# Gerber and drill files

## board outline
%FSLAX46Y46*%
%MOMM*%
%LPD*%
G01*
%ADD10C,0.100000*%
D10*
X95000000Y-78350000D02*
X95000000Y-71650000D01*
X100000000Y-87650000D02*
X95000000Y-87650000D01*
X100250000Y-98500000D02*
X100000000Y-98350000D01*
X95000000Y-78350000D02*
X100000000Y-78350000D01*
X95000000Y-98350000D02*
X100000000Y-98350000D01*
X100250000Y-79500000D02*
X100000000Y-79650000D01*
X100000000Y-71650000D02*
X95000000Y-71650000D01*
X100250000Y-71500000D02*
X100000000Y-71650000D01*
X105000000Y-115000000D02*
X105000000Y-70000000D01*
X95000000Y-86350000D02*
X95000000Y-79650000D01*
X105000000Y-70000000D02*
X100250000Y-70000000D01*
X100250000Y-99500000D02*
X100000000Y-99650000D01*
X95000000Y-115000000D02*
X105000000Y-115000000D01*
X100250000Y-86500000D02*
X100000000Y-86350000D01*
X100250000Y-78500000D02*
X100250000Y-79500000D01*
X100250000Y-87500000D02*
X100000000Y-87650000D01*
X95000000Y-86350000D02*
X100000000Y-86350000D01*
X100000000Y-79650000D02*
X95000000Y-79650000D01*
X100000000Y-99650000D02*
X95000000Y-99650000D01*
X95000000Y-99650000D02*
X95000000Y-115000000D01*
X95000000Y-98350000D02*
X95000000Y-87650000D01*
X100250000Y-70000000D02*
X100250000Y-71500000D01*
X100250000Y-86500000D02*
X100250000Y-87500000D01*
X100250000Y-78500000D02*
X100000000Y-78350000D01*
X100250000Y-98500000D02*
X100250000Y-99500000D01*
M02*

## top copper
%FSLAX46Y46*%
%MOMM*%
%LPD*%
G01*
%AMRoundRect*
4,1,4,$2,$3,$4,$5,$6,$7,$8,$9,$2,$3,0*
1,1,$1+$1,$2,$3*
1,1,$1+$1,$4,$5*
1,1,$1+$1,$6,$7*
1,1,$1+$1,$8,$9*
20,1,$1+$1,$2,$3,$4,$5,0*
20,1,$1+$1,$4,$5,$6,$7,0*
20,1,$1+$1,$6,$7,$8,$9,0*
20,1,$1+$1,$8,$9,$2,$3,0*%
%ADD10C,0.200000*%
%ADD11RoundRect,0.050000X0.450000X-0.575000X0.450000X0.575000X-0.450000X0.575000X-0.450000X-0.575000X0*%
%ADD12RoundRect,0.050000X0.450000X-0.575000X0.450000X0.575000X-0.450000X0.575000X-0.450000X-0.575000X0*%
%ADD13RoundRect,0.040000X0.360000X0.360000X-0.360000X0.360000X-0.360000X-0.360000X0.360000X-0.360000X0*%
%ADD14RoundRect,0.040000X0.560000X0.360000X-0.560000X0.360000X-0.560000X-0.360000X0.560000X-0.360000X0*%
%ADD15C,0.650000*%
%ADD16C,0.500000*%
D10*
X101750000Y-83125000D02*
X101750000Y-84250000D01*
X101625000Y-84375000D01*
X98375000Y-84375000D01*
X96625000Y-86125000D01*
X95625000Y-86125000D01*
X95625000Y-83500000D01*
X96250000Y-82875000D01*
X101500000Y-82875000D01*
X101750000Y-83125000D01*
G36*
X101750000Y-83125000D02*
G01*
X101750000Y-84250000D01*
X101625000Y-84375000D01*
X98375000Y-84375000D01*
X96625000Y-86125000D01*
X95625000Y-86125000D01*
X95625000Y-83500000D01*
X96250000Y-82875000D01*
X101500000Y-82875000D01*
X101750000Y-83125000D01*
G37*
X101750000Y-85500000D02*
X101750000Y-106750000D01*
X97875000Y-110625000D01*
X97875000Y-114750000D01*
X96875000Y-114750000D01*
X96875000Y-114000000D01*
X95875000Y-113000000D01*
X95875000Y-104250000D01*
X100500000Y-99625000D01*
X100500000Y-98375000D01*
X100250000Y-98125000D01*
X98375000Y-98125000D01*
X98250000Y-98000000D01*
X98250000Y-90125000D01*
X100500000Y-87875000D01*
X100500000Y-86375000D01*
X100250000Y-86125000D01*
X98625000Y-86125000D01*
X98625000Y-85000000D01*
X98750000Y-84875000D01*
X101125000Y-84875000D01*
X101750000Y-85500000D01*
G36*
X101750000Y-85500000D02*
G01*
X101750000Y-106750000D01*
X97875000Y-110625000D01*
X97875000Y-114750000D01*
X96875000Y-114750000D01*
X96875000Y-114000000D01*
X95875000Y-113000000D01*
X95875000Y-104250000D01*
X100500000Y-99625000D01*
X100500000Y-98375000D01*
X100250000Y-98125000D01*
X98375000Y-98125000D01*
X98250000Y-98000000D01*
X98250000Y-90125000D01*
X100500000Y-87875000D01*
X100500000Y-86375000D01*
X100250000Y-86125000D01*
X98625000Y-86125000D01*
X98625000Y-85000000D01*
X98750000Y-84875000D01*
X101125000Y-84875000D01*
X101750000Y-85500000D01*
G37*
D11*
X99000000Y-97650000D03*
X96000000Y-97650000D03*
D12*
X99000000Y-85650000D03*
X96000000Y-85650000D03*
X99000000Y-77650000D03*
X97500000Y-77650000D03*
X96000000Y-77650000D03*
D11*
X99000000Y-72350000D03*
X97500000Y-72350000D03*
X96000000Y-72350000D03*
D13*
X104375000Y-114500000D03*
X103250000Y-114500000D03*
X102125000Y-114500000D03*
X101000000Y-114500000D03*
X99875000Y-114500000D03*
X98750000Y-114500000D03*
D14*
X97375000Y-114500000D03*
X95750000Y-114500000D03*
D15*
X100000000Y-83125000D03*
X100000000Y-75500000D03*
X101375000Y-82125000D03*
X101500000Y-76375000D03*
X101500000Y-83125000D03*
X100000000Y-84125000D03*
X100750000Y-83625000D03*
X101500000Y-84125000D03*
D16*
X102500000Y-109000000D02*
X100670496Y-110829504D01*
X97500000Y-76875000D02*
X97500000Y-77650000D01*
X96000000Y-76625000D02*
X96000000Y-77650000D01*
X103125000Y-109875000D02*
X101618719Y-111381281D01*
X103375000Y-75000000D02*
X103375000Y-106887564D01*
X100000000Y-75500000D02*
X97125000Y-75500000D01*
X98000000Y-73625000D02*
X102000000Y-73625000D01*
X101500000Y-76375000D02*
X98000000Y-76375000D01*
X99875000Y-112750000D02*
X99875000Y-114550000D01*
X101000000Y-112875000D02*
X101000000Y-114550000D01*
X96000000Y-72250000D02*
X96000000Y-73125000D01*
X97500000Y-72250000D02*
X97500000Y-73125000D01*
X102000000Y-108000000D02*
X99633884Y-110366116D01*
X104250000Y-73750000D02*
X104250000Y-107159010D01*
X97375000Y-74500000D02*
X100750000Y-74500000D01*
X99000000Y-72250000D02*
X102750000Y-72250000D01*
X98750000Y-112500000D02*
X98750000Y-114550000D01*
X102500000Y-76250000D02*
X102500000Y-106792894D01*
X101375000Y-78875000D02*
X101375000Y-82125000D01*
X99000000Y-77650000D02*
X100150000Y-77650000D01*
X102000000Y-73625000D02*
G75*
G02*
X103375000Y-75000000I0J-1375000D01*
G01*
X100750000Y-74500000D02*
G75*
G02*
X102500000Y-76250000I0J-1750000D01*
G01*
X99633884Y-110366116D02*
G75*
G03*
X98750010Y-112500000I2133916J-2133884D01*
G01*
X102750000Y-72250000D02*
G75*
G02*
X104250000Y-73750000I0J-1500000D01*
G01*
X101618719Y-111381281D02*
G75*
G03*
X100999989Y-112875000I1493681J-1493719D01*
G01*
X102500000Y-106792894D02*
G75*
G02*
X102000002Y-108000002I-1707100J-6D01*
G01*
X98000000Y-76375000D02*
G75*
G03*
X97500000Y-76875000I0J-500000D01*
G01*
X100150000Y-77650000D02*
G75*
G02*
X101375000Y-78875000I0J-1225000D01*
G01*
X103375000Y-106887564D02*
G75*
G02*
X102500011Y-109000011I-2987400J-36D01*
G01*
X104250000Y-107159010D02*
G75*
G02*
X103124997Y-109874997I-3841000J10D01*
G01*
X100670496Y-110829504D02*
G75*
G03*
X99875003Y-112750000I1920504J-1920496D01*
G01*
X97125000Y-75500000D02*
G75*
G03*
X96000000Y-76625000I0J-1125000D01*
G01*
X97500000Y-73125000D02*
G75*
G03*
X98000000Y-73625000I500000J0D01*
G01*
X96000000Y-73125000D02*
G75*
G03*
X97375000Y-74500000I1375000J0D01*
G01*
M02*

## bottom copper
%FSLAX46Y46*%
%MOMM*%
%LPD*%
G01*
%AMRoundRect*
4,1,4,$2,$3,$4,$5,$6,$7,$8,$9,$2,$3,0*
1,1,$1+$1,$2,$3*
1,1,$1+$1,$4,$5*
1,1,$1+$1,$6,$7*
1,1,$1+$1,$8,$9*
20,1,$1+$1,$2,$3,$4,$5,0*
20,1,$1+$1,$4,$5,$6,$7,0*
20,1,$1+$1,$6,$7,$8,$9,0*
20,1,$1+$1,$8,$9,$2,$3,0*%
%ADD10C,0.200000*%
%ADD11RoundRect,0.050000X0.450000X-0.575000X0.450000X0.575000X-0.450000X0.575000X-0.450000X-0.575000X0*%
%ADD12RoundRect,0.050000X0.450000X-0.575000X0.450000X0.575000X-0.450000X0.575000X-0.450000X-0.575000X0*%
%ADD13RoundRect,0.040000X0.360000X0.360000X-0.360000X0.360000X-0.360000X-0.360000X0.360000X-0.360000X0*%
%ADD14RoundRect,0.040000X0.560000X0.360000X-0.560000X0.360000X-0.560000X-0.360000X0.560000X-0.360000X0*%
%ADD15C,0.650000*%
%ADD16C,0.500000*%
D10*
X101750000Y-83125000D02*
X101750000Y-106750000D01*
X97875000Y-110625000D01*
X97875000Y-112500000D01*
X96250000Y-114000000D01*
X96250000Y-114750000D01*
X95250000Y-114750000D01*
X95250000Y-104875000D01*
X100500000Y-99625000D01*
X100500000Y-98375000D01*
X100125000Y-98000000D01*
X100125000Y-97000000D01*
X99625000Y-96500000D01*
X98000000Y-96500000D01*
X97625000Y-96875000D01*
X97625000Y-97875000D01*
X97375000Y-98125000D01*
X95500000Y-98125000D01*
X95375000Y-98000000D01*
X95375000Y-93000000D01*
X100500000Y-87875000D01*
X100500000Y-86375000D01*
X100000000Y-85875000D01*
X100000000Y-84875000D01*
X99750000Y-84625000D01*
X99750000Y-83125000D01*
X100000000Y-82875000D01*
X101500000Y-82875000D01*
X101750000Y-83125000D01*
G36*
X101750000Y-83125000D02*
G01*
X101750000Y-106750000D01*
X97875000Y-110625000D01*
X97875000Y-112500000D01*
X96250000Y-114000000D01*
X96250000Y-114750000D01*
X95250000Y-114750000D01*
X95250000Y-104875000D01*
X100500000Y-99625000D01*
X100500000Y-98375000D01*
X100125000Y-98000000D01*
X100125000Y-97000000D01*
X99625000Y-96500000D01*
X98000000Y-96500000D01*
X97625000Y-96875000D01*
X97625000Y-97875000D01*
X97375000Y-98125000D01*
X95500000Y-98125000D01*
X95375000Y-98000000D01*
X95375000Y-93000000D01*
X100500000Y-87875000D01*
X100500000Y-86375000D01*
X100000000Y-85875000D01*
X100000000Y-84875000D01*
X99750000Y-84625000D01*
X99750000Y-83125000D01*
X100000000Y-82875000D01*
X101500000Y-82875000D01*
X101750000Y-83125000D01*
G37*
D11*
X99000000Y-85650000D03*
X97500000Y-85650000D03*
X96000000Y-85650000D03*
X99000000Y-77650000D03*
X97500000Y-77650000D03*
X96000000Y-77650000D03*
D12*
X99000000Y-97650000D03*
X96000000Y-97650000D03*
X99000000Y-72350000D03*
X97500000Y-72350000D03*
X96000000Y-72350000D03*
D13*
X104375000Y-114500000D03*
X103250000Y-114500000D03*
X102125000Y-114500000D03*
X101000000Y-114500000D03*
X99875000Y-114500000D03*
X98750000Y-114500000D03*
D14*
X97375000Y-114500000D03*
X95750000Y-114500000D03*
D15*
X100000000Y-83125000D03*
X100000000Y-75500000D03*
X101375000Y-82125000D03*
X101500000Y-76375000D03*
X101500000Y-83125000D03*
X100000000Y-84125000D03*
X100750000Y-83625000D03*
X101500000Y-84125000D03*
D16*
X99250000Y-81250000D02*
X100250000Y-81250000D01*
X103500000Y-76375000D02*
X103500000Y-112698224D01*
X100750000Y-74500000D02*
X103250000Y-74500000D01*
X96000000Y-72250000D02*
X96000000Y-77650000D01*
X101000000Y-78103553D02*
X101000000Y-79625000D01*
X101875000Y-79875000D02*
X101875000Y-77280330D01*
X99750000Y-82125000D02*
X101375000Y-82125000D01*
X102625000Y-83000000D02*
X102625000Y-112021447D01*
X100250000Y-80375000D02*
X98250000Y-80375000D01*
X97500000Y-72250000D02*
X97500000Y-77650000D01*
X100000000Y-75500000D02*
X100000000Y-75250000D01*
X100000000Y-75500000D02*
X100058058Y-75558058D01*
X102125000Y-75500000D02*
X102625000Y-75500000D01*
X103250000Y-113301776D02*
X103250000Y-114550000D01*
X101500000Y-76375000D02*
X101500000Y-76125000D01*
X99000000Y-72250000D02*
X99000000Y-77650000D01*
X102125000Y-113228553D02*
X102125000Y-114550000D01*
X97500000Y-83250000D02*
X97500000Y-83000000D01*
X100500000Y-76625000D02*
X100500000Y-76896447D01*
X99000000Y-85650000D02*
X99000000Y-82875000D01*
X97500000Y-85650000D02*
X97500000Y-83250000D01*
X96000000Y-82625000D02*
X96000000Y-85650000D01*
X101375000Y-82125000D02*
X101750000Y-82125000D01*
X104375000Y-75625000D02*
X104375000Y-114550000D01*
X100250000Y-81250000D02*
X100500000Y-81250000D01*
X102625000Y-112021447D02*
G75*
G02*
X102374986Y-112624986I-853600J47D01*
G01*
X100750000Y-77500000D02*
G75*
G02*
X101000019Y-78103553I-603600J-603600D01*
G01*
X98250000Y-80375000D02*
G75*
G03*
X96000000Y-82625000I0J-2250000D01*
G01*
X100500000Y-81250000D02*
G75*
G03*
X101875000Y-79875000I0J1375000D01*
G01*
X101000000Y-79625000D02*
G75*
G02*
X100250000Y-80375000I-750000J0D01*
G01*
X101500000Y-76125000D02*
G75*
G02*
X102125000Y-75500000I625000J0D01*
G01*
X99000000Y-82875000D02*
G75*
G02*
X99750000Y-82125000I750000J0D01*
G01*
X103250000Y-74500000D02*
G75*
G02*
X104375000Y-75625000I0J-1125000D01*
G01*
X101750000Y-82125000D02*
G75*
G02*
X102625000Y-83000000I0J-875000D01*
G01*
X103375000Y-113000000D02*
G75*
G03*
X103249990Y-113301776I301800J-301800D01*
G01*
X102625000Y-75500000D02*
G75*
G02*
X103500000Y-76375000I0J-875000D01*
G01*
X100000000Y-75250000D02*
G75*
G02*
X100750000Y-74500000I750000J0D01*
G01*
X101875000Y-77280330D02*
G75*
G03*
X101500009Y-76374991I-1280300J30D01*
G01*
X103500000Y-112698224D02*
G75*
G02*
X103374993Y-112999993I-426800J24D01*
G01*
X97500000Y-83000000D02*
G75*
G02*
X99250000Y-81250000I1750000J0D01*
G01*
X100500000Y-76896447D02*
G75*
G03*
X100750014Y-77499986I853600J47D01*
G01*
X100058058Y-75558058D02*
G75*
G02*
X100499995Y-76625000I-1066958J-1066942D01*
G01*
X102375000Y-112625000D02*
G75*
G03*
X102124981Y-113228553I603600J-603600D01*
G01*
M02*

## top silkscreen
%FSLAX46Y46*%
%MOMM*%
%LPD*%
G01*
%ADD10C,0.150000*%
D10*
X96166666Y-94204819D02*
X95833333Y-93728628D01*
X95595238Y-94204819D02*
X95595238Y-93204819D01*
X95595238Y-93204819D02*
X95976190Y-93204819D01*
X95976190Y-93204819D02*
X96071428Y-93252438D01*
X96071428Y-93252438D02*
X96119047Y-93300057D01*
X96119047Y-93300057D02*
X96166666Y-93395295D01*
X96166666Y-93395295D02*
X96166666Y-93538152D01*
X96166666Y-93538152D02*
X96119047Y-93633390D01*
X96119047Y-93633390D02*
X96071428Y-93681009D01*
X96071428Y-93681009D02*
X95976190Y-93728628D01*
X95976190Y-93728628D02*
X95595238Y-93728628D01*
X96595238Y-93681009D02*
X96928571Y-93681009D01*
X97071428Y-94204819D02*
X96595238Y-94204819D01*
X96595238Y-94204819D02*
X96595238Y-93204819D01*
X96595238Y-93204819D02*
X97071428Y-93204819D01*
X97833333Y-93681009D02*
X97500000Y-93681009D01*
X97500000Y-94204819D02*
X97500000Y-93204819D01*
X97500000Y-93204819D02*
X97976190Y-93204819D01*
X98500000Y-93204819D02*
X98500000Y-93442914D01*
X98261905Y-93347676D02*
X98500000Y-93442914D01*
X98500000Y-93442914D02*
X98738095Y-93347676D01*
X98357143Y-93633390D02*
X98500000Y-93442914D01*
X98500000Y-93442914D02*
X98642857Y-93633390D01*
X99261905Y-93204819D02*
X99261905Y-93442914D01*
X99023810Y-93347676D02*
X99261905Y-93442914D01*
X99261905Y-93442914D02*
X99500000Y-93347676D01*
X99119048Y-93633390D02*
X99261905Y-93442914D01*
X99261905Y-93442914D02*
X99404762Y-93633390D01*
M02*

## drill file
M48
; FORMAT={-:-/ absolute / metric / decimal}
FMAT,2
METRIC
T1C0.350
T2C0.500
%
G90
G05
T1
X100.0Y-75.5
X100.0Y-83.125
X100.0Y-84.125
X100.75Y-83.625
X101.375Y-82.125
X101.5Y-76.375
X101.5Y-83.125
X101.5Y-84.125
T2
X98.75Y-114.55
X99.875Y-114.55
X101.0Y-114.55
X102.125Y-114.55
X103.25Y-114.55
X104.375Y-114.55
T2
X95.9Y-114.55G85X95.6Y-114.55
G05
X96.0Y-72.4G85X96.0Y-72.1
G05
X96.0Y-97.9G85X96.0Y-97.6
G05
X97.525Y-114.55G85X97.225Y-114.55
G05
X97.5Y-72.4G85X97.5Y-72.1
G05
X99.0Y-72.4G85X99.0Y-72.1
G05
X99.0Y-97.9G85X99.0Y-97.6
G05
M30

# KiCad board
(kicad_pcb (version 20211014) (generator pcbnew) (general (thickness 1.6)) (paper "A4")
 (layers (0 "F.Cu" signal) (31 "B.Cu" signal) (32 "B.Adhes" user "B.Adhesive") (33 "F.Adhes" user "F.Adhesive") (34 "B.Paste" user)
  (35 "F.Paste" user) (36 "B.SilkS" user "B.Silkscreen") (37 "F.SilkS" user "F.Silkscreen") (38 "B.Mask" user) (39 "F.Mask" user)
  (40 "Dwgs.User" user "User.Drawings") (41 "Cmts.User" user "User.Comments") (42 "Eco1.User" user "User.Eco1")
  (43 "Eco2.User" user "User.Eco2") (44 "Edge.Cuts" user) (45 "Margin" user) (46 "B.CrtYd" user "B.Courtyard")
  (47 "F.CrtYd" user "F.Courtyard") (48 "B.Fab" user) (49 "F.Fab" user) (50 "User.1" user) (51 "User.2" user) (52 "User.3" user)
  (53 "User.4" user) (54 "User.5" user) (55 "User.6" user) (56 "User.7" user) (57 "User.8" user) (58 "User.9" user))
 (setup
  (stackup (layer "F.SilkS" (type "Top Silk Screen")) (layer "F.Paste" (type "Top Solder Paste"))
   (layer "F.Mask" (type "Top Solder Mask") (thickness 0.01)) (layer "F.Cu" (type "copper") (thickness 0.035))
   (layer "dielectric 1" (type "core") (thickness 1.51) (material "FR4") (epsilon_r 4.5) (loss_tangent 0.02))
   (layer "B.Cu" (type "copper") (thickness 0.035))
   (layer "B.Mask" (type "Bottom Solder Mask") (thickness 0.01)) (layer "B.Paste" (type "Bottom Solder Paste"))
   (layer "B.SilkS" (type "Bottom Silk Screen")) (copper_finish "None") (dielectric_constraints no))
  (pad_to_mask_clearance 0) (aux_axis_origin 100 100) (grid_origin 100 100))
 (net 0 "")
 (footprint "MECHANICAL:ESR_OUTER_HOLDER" (layer "F.Cu") (at 100 100)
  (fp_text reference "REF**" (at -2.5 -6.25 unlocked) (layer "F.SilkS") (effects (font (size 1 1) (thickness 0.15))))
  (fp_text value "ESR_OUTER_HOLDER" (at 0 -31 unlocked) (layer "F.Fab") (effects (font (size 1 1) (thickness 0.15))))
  (fp_line (start -5 -21.65) (end -5 -28.35) (layer "Edge.Cuts") (width 0.1))
  (fp_line (start 0 -12.35) (end -5 -12.35) (layer "Edge.Cuts") (width 0.1))
  (fp_line (start 0.25 -1.5) (end 0 -1.65) (layer "Edge.Cuts") (width 0.1))
  (fp_line (start -5 -21.65) (end 0 -21.65) (layer "Edge.Cuts") (width 0.1))
  (fp_line (start -5 -1.65) (end 0 -1.65) (layer "Edge.Cuts") (width 0.1))
  (fp_line (start 0.25 -20.5) (end 0 -20.35) (layer "Edge.Cuts") (width 0.1))
  (fp_line (start 0 -28.35) (end -5 -28.35) (layer "Edge.Cuts") (width 0.1))
  (fp_line (start 0.25 -28.5) (end 0 -28.35) (layer "Edge.Cuts") (width 0.1))
  (fp_line (start 5 15) (end 5 -30) (layer "Edge.Cuts") (width 0.1))
  (fp_line (start -5 -13.65) (end -5 -20.35) (layer "Edge.Cuts") (width 0.1))
  (fp_line (start 5 -30) (end 0.25 -30) (layer "Edge.Cuts") (width 0.1))
  (fp_line (start 0.25 -0.5) (end 0 -0.35) (layer "Edge.Cuts") (width 0.1))
  (fp_line (start -5 15) (end 5 15) (layer "Edge.Cuts") (width 0.1))
  (fp_line (start 0.25 -13.5) (end 0 -13.65) (layer "Edge.Cuts") (width 0.1))
  (fp_line (start 0.25 -21.5) (end 0.25 -20.5) (layer "Edge.Cuts") (width 0.1))
  (fp_line (start 0.25 -12.5) (end 0 -12.35) (layer "Edge.Cuts") (width 0.1))
  (fp_line (start -5 -13.65) (end 0 -13.65) (layer "Edge.Cuts") (width 0.1))
  (fp_line (start 0 -20.35) (end -5 -20.35) (layer "Edge.Cuts") (width 0.1))
  (fp_line (start 0 -0.35) (end -5 -0.35) (layer "Edge.Cuts") (width 0.1))
  (fp_line (start -5 -0.35) (end -5 15) (layer "Edge.Cuts") (width 0.1))
  (fp_line (start -5 -1.65) (end -5 -12.35) (layer "Edge.Cuts") (width 0.1))
  (fp_line (start 0.25 -30) (end 0.25 -28.5) (layer "Edge.Cuts") (width 0.1))
  (fp_line (start 0.25 -13.5) (end 0.25 -12.5) (layer "Edge.Cuts") (width 0.1))
  (fp_line (start 0.25 -21.5) (end 0 -21.65) (layer "Edge.Cuts") (width 0.1))
  (fp_line (start 0.25 -1.5) (end 0.25 -0.5) (layer "Edge.Cuts") (width 0.1))
  (pad "*4" smd roundrect (at -1 -14.35 90) (size 1.25 1) (layers "B.Cu" "B.Paste" "B.Mask") (roundrect_rratio 0.05)
   (solder_mask_margin 0.05) (solder_paste_margin_ratio -0.1))
  (pad "*5" smd roundrect (at -2.5 -14.35 90) (size 1.25 1) (layers "B.Cu" "B.Paste" "B.Mask") (roundrect_rratio 0.05)
   (solder_mask_margin 0.05) (solder_paste_margin_ratio -0.1))
  (pad "*6" smd roundrect (at -4 -14.35 90) (size 1.25 1) (layers "B.Cu" "B.Paste" "B.Mask") (roundrect_rratio 0.05)
   (solder_mask_margin 0.05) (solder_paste_margin_ratio -0.1))
  (pad "*7" smd roundrect (at -1 -22.35 90) (size 1.25 1) (layers "B.Cu" "B.Paste" "B.Mask") (roundrect_rratio 0.05)
   (solder_mask_margin 0.05) (solder_paste_margin_ratio -0.1))
  (pad "*8" smd roundrect (at -2.5 -22.35 90) (size 1.25 1) (layers "B.Cu" "B.Paste" "B.Mask") (roundrect_rratio 0.05)
   (solder_mask_margin 0.05) (solder_paste_margin_ratio -0.1))
  (pad "*9" smd roundrect (at -4 -22.35 90) (size 1.25 1) (layers "B.Cu" "B.Paste" "B.Mask") (roundrect_rratio 0.05)
   (solder_mask_margin 0.05) (solder_paste_margin_ratio -0.1))
  (pad "1" thru_hole roundrect (at -1 -2.25 90) (size 1.25 1) (drill oval 0.8 0.5 (offset 0.1 0)) (layers *.Cu *.Mask)
   (roundrect_rratio 0.05) (solder_mask_margin 0.05) (solder_paste_margin_ratio -0.1))
  (pad "3" thru_hole roundrect (at -4 -2.25 90) (size 1.25 1) (drill oval 0.8 0.5 (offset 0.1 0)) (layers *.Cu *.Mask)
   (roundrect_rratio 0.05) (solder_mask_margin 0.05) (solder_paste_margin_ratio -0.1))
  (pad "4" smd roundrect (at -1 -14.35 90) (size 1.25 1) (layers "F.Cu" "F.Paste" "F.Mask") (roundrect_rratio 0.05)
   (solder_mask_margin 0.05) (solder_paste_margin_ratio -0.1))
  (pad "6" smd roundrect (at -4 -14.35 90) (size 1.25 1) (layers "F.Cu" "F.Paste" "F.Mask") (roundrect_rratio 0.05)
   (solder_mask_margin 0.05) (solder_paste_margin_ratio -0.1))
  (pad "7" smd roundrect (at -1 -22.35 90) (size 1.25 1) (layers "F.Cu" "F.Paste" "F.Mask") (roundrect_rratio 0.05)
   (solder_mask_margin 0.05) (solder_paste_margin_ratio -0.1))
  (pad "8" smd roundrect (at -2.5 -22.35 90) (size 1.25 1) (layers "F.Cu" "F.Paste" "F.Mask") (roundrect_rratio 0.05)
   (solder_mask_margin 0.05) (solder_paste_margin_ratio -0.1))
  (pad "9" smd roundrect (at -4 -22.35 90) (size 1.25 1) (layers "F.Cu" "F.Paste" "F.Mask") (roundrect_rratio 0.05)
   (solder_mask_margin 0.05) (solder_paste_margin_ratio -0.1))
  (pad "10" thru_hole roundrect (at -1 -27.75 90) (size 1.25 1) (drill oval 0.8 0.5 (offset -0.1 0)) (layers *.Cu *.Mask)
   (roundrect_rratio 0.05) (solder_mask_margin 0.05) (solder_paste_margin_ratio -0.1))
  (pad "11" thru_hole roundrect (at -2.5 -27.75 90) (size 1.25 1) (drill oval 0.8 0.5 (offset -0.1 0)) (layers *.Cu *.Mask)
   (roundrect_rratio 0.05) (solder_mask_margin 0.05) (solder_paste_margin_ratio -0.1))
  (pad "12" thru_hole roundrect (at -4 -27.75 90) (size 1.25 1) (drill oval 0.8 0.5 (offset -0.1 0)) (layers *.Cu *.Mask)
   (roundrect_rratio 0.05) (solder_mask_margin 0.05) (solder_paste_margin_ratio -0.1))
  (pad "A" thru_hole roundrect (at 4.375 14.55 180) (size 0.8 0.8) (drill 0.5 (offset 0 0.05)) (layers *.Cu *.Mask) (roundrect_rratio 0.05)
   (solder_mask_margin 0.05) (solder_paste_margin_ratio -0.1))
  (pad "B" thru_hole roundrect (at 3.25 14.55 180) (size 0.8 0.8) (drill 0.5 (offset 0 0.05)) (layers *.Cu *.Mask) (roundrect_rratio 0.05)
   (solder_mask_margin 0.05) (solder_paste_margin_ratio -0.1))
  (pad "C" thru_hole roundrect (at 2.125 14.55 180) (size 0.8 0.8) (drill 0.5 (offset 0 0.05)) (layers *.Cu *.Mask) (roundrect_rratio 0.05)
   (solder_mask_margin 0.05) (solder_paste_margin_ratio -0.1))
  (pad "D" thru_hole roundrect (at 1 14.55 180) (size 0.8 0.8) (drill 0.5 (offset 0 0.05)) (layers *.Cu *.Mask) (roundrect_rratio 0.05)
   (solder_mask_margin 0.05) (solder_paste_margin_ratio -0.1))
  (pad "E" thru_hole roundrect (at -0.125 14.55 180) (size 0.8 0.8) (drill 0.5 (offset 0 0.05)) (layers *.Cu *.Mask) (roundrect_rratio 0.05)
   (solder_mask_margin 0.05) (solder_paste_margin_ratio -0.1))
  (pad "F" thru_hole roundrect (at -1.25 14.55 180) (size 0.8 0.8) (drill 0.5 (offset 0 0.05)) (layers *.Cu *.Mask) (roundrect_rratio 0.05)
   (solder_mask_margin 0.05) (solder_paste_margin_ratio -0.1))
  (pad "G" thru_hole roundrect (at -2.625 14.55 180) (size 1.2 0.8) (drill oval 0.8 0.5 (offset 0 0.05)) (layers *.Cu *.Mask)
   (roundrect_rratio 0.05) (solder_mask_margin 0.05) (solder_paste_margin_ratio -0.1))
  (pad "H" thru_hole roundrect (at -4.25 14.55 180) (size 1.2 0.8) (drill oval 0.8 0.5 (offset 0 0.05)) (layers *.Cu *.Mask)
   (roundrect_rratio 0.05) (solder_mask_margin 0.05) (solder_paste_margin_ratio -0.1)))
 (gr_poly
  (pts (xy 101.75 83.125) (xy 101.75 84.25) (xy 101.625 84.375) (xy 98.375 84.375) (xy 96.625 86.125) (xy 95.625 86.125) (xy 95.625 83.5)
   (xy 96.25 82.875) (xy 101.5 82.875))
  (layer "F.Cu") (width 0.2) (fill solid))
 (gr_poly
  (pts (xy 101.75 85.5) (xy 101.75 106.75) (xy 97.875 110.625) (xy 97.875 114.75) (xy 96.875 114.75) (xy 96.875 114) (xy 95.875 113)
   (xy 95.875 104.25) (xy 100.5 99.625) (xy 100.5 98.375) (xy 100.25 98.125) (xy 98.375 98.125) (xy 98.25 98) (xy 98.25 90.125)
   (xy 100.5 87.875) (xy 100.5 86.375) (xy 100.25 86.125) (xy 98.625 86.125) (xy 98.625 85) (xy 98.75 84.875) (xy 101.125 84.875))
  (layer "F.Cu") (width 0.2) (fill solid))
 (gr_poly
  (pts (xy 101.75 83.125) (xy 101.75 106.75) (xy 97.875 110.625) (xy 97.875 112.5) (xy 96.25 114) (xy 96.25 114.75) (xy 95.25 114.75)
   (xy 95.25 104.875) (xy 100.5 99.625) (xy 100.5 98.375) (xy 100.125 98) (xy 100.125 97) (xy 99.625 96.5) (xy 98 96.5) (xy 97.625 96.875)
   (xy 97.625 97.875) (xy 97.375 98.125) (xy 95.5 98.125) (xy 95.375 98) (xy 95.375 93) (xy 100.5 87.875) (xy 100.5 86.375) (xy 100 85.875)
   (xy 100 84.875) (xy 99.75 84.625) (xy 99.75 83.125) (xy 100 82.875) (xy 101.5 82.875))
  (layer "B.Cu") (width 0.2) (fill solid))
 (segment (start 102.5 109) (end 100.670496 110.829504) (width 0.5) (layer "F.Cu") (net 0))
 (segment (start 97.5 76.875) (end 97.5 77.65) (width 0.5) (layer "F.Cu") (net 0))
 (segment (start 96 76.625) (end 96 77.65) (width 0.5) (layer "F.Cu") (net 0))
 (segment (start 103.125 109.875) (end 101.618719 111.381281) (width 0.5) (layer "F.Cu") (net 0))
 (segment (start 103.375 75) (end 103.375 106.887564) (width 0.5) (layer "F.Cu") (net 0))
 (segment (start 100 75.5) (end 97.125 75.5) (width 0.5) (layer "F.Cu") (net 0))
 (segment (start 98 73.625) (end 102 73.625) (width 0.5) (layer "F.Cu") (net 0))
 (segment (start 101.5 76.375) (end 98 76.375) (width 0.5) (layer "F.Cu") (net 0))
 (segment (start 99.875 112.75) (end 99.875 114.55) (width 0.5) (layer "F.Cu") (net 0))
 (segment (start 101 112.875) (end 101 114.55) (width 0.5) (layer "F.Cu") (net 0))
 (segment (start 96 72.25) (end 96 73.125) (width 0.5) (layer "F.Cu") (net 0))
 (segment (start 97.5 72.25) (end 97.5 73.125) (width 0.5) (layer "F.Cu") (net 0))
 (segment (start 102 108) (end 99.633884 110.366116) (width 0.5) (layer "F.Cu") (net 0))
 (segment (start 104.25 73.75) (end 104.25 107.15901) (width 0.5) (layer "F.Cu") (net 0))
 (segment (start 97.375 74.5) (end 100.75 74.5) (width 0.5) (layer "F.Cu") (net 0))
 (segment (start 99 72.25) (end 102.75 72.25) (width 0.5) (layer "F.Cu") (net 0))
 (segment (start 98.75 112.5) (end 98.75 114.55) (width 0.5) (layer "F.Cu") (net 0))
 (segment (start 102.5 76.25) (end 102.5 106.792894) (width 0.5) (layer "F.Cu") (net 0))
 (segment (start 101.375 78.875) (end 101.375 82.125) (width 0.5) (layer "F.Cu") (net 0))
 (segment (start 99 77.65) (end 100.15 77.65) (width 0.5) (layer "F.Cu") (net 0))
 (via (at 100 83.125) (size 0.65) (drill 0.35) (layers "F.Cu" "B.Cu") (free) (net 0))
 (via (at 100 75.5) (size 0.65) (drill 0.35) (layers "F.Cu" "B.Cu") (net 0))
 (via (at 101.375 82.125) (size 0.65) (drill 0.35) (layers "F.Cu" "B.Cu") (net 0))
 (via (at 101.5 76.375) (size 0.65) (drill 0.35) (layers "F.Cu" "B.Cu") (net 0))
 (via (at 101.5 83.125) (size 0.65) (drill 0.35) (layers "F.Cu" "B.Cu") (free) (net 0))
 (via (at 100 84.125) (size 0.65) (drill 0.35) (layers "F.Cu" "B.Cu") (free) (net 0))
 (via (at 100.75 83.625) (size 0.65) (drill 0.35) (layers "F.Cu" "B.Cu") (free) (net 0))
 (via (at 101.5 84.125) (size 0.65) (drill 0.35) (layers "F.Cu" "B.Cu") (free) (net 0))
 (arc (start 102 73.625) (mid 102.972272 74.027728) (end 103.375 75) (width 0.5) (layer "F.Cu") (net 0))
 (arc (start 100.75 74.5) (mid 101.987437 75.012563) (end 102.5 76.25) (width 0.5) (layer "F.Cu") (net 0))
 (arc (start 99.633884 110.366116) (mid 98.979714 111.34515) (end 98.75 112.5) (width 0.5) (layer "F.Cu") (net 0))
 (arc (start 102.75 72.25) (mid 103.81066 72.68934) (end 104.25 73.75) (width 0.5) (layer "F.Cu") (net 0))
 (arc (start 101.618719 111.381281) (mid 101.1608 112.066605) (end 101 112.875) (width 0.5) (layer "F.Cu") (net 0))
 (arc (start 102.5 106.792894) (mid 102.370054 107.446175) (end 102 108) (width 0.5) (layer "F.Cu") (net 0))
 (arc (start 98 76.375) (mid 97.646447 76.521447) (end 97.5 76.875) (width 0.5) (layer "F.Cu") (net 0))
 (arc (start 100.15 77.65) (mid 101.016206 78.008794) (end 101.375 78.875) (width 0.5) (layer "F.Cu") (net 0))
 (arc (start 103.375 106.887564) (mid 103.147595 108.030806) (end 102.5 109) (width 0.5) (layer "F.Cu") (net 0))
 (arc (start 104.25 107.15901) (mid 103.957622 108.628893) (end 103.125 109.875) (width 0.5) (layer "F.Cu") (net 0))
 (arc (start 100.670496 110.829504) (mid 100.081743 111.710635) (end 99.875 112.75) (width 0.5) (layer "F.Cu") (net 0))
 (arc (start 97.125 75.5) (mid 96.329505 75.829505) (end 96 76.625) (width 0.5) (layer "F.Cu") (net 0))
 (arc (start 97.5 73.125) (mid 97.646447 73.478553) (end 98 73.625) (width 0.5) (layer "F.Cu") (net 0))
 (arc (start 96 73.125) (mid 96.402728 74.097272) (end 97.375 74.5) (width 0.5) (layer "F.Cu") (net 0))
 (segment (start 99.25 81.25) (end 100.25 81.25) (width 0.5) (layer "B.Cu") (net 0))
 (segment (start 103.5 76.375) (end 103.5 112.698224) (width 0.5) (layer "B.Cu") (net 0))
 (segment (start 100.75 74.5) (end 103.25 74.5) (width 0.5) (layer "B.Cu") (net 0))
 (segment (start 96 72.25) (end 96 77.65) (width 0.5) (layer "B.Cu") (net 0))
 (segment (start 101 78.103553) (end 101 79.625) (width 0.5) (layer "B.Cu") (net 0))
 (segment (start 101.875 79.875) (end 101.875 77.28033) (width 0.5) (layer "B.Cu") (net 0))
 (segment (start 99.75 82.125) (end 101.375 82.125) (width 0.5) (layer "B.Cu") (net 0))
 (segment (start 102.625 83) (end 102.625 112.021447) (width 0.5) (layer "B.Cu") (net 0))
 (segment (start 100.25 80.375) (end 98.25 80.375) (width 0.5) (layer "B.Cu") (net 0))
 (segment (start 97.5 72.25) (end 97.5 77.65) (width 0.5) (layer "B.Cu") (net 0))
 (segment (start 100 75.5) (end 100 75.25) (width 0.5) (layer "B.Cu") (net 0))
 (segment (start 100 75.5) (end 100.058058 75.558058) (width 0.5) (layer "B.Cu") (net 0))
 (segment (start 102.125 75.5) (end 102.625 75.5) (width 0.5) (layer "B.Cu") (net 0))
 (segment (start 103.25 113.301776) (end 103.25 114.55) (width 0.5) (layer "B.Cu") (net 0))
 (segment (start 101.5 76.375) (end 101.5 76.125) (width 0.5) (layer "B.Cu") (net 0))
 (segment (start 99 72.25) (end 99 77.65) (width 0.5) (layer "B.Cu") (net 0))
 (segment (start 102.125 113.228553) (end 102.125 114.55) (width 0.5) (layer "B.Cu") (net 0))
 (segment (start 97.5 83.25) (end 97.5 83) (width 0.5) (layer "B.Cu") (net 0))
 (segment (start 100.5 76.625) (end 100.5 76.896447) (width 0.5) (layer "B.Cu") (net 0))
 (segment (start 99 85.65) (end 99 82.875) (width 0.5) (layer "B.Cu") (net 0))
 (segment (start 97.5 85.65) (end 97.5 83.25) (width 0.5) (layer "B.Cu") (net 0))
 (segment (start 96 82.625) (end 96 85.65) (width 0.5) (layer "B.Cu") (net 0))
 (segment (start 101.375 82.125) (end 101.75 82.125) (width 0.5) (layer "B.Cu") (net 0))
 (segment (start 104.375 75.625) (end 104.375 114.55) (width 0.5) (layer "B.Cu") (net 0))
 (segment (start 100.25 81.25) (end 100.5 81.25) (width 0.5) (layer "B.Cu") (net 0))
 (arc (start 102.625 112.021447) (mid 102.560027 112.348088) (end 102.375 112.625) (width 0.5) (layer "B.Cu") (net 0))
 (arc (start 100.75 77.5) (mid 100.935027 77.776912) (end 101 78.103553) (width 0.5) (layer "B.Cu") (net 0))
 (arc (start 98.25 80.375) (mid 96.65901 81.03401) (end 96 82.625) (width 0.5) (layer "B.Cu") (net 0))
 (arc (start 100.5 81.25) (mid 101.472272 80.847272) (end 101.875 79.875) (width 0.5) (layer "B.Cu") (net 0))
 (arc (start 101 79.625) (mid 100.78033 80.15533) (end 100.25 80.375) (width 0.5) (layer "B.Cu") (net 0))
 (arc (start 101.5 76.125) (mid 101.683058 75.683058) (end 102.125 75.5) (width 0.5) (layer "B.Cu") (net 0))
 (arc (start 99 82.875) (mid 99.21967 82.34467) (end 99.75 82.125) (width 0.5) (layer "B.Cu") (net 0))
 (arc (start 103.25 74.5) (mid 104.045495 74.829505) (end 104.375 75.625) (width 0.5) (layer "B.Cu") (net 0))
 (arc (start 101.75 82.125) (mid 102.368718 82.381282) (end 102.625 83) (width 0.5) (layer "B.Cu") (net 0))
 (arc (start 103.375 113) (mid 103.282487 113.138456) (end 103.25 113.301776) (width 0.5) (layer "B.Cu") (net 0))
 (arc (start 102.625 75.5) (mid 103.243718 75.756282) (end 103.5 76.375) (width 0.5) (layer "B.Cu") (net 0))
 (arc (start 100 75.25) (mid 100.21967 74.71967) (end 100.75 74.5) (width 0.5) (layer "B.Cu") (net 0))
 (arc (start 101.875 77.28033) (mid 101.777541 76.790369) (end 101.5 76.375) (width 0.5) (layer "B.Cu") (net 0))
 (arc (start 103.5 112.698224) (mid 103.467513 112.861544) (end 103.375 113) (width 0.5) (layer "B.Cu") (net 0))
 (arc (start 97.5 83) (mid 98.012563 81.762563) (end 99.25 81.25) (width 0.5) (layer "B.Cu") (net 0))
 (arc (start 100.5 76.896447) (mid 100.564973 77.223087) (end 100.75 77.5) (width 0.5) (layer "B.Cu") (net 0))
 (arc (start 100.058058 75.558058) (mid 100.385143 76.047575) (end 100.5 76.625) (width 0.5) (layer "B.Cu") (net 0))
 (arc (start 102.375 112.625) (mid 102.189973 112.901912) (end 102.125 113.228553) (width 0.5) (layer "B.Cu") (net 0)))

